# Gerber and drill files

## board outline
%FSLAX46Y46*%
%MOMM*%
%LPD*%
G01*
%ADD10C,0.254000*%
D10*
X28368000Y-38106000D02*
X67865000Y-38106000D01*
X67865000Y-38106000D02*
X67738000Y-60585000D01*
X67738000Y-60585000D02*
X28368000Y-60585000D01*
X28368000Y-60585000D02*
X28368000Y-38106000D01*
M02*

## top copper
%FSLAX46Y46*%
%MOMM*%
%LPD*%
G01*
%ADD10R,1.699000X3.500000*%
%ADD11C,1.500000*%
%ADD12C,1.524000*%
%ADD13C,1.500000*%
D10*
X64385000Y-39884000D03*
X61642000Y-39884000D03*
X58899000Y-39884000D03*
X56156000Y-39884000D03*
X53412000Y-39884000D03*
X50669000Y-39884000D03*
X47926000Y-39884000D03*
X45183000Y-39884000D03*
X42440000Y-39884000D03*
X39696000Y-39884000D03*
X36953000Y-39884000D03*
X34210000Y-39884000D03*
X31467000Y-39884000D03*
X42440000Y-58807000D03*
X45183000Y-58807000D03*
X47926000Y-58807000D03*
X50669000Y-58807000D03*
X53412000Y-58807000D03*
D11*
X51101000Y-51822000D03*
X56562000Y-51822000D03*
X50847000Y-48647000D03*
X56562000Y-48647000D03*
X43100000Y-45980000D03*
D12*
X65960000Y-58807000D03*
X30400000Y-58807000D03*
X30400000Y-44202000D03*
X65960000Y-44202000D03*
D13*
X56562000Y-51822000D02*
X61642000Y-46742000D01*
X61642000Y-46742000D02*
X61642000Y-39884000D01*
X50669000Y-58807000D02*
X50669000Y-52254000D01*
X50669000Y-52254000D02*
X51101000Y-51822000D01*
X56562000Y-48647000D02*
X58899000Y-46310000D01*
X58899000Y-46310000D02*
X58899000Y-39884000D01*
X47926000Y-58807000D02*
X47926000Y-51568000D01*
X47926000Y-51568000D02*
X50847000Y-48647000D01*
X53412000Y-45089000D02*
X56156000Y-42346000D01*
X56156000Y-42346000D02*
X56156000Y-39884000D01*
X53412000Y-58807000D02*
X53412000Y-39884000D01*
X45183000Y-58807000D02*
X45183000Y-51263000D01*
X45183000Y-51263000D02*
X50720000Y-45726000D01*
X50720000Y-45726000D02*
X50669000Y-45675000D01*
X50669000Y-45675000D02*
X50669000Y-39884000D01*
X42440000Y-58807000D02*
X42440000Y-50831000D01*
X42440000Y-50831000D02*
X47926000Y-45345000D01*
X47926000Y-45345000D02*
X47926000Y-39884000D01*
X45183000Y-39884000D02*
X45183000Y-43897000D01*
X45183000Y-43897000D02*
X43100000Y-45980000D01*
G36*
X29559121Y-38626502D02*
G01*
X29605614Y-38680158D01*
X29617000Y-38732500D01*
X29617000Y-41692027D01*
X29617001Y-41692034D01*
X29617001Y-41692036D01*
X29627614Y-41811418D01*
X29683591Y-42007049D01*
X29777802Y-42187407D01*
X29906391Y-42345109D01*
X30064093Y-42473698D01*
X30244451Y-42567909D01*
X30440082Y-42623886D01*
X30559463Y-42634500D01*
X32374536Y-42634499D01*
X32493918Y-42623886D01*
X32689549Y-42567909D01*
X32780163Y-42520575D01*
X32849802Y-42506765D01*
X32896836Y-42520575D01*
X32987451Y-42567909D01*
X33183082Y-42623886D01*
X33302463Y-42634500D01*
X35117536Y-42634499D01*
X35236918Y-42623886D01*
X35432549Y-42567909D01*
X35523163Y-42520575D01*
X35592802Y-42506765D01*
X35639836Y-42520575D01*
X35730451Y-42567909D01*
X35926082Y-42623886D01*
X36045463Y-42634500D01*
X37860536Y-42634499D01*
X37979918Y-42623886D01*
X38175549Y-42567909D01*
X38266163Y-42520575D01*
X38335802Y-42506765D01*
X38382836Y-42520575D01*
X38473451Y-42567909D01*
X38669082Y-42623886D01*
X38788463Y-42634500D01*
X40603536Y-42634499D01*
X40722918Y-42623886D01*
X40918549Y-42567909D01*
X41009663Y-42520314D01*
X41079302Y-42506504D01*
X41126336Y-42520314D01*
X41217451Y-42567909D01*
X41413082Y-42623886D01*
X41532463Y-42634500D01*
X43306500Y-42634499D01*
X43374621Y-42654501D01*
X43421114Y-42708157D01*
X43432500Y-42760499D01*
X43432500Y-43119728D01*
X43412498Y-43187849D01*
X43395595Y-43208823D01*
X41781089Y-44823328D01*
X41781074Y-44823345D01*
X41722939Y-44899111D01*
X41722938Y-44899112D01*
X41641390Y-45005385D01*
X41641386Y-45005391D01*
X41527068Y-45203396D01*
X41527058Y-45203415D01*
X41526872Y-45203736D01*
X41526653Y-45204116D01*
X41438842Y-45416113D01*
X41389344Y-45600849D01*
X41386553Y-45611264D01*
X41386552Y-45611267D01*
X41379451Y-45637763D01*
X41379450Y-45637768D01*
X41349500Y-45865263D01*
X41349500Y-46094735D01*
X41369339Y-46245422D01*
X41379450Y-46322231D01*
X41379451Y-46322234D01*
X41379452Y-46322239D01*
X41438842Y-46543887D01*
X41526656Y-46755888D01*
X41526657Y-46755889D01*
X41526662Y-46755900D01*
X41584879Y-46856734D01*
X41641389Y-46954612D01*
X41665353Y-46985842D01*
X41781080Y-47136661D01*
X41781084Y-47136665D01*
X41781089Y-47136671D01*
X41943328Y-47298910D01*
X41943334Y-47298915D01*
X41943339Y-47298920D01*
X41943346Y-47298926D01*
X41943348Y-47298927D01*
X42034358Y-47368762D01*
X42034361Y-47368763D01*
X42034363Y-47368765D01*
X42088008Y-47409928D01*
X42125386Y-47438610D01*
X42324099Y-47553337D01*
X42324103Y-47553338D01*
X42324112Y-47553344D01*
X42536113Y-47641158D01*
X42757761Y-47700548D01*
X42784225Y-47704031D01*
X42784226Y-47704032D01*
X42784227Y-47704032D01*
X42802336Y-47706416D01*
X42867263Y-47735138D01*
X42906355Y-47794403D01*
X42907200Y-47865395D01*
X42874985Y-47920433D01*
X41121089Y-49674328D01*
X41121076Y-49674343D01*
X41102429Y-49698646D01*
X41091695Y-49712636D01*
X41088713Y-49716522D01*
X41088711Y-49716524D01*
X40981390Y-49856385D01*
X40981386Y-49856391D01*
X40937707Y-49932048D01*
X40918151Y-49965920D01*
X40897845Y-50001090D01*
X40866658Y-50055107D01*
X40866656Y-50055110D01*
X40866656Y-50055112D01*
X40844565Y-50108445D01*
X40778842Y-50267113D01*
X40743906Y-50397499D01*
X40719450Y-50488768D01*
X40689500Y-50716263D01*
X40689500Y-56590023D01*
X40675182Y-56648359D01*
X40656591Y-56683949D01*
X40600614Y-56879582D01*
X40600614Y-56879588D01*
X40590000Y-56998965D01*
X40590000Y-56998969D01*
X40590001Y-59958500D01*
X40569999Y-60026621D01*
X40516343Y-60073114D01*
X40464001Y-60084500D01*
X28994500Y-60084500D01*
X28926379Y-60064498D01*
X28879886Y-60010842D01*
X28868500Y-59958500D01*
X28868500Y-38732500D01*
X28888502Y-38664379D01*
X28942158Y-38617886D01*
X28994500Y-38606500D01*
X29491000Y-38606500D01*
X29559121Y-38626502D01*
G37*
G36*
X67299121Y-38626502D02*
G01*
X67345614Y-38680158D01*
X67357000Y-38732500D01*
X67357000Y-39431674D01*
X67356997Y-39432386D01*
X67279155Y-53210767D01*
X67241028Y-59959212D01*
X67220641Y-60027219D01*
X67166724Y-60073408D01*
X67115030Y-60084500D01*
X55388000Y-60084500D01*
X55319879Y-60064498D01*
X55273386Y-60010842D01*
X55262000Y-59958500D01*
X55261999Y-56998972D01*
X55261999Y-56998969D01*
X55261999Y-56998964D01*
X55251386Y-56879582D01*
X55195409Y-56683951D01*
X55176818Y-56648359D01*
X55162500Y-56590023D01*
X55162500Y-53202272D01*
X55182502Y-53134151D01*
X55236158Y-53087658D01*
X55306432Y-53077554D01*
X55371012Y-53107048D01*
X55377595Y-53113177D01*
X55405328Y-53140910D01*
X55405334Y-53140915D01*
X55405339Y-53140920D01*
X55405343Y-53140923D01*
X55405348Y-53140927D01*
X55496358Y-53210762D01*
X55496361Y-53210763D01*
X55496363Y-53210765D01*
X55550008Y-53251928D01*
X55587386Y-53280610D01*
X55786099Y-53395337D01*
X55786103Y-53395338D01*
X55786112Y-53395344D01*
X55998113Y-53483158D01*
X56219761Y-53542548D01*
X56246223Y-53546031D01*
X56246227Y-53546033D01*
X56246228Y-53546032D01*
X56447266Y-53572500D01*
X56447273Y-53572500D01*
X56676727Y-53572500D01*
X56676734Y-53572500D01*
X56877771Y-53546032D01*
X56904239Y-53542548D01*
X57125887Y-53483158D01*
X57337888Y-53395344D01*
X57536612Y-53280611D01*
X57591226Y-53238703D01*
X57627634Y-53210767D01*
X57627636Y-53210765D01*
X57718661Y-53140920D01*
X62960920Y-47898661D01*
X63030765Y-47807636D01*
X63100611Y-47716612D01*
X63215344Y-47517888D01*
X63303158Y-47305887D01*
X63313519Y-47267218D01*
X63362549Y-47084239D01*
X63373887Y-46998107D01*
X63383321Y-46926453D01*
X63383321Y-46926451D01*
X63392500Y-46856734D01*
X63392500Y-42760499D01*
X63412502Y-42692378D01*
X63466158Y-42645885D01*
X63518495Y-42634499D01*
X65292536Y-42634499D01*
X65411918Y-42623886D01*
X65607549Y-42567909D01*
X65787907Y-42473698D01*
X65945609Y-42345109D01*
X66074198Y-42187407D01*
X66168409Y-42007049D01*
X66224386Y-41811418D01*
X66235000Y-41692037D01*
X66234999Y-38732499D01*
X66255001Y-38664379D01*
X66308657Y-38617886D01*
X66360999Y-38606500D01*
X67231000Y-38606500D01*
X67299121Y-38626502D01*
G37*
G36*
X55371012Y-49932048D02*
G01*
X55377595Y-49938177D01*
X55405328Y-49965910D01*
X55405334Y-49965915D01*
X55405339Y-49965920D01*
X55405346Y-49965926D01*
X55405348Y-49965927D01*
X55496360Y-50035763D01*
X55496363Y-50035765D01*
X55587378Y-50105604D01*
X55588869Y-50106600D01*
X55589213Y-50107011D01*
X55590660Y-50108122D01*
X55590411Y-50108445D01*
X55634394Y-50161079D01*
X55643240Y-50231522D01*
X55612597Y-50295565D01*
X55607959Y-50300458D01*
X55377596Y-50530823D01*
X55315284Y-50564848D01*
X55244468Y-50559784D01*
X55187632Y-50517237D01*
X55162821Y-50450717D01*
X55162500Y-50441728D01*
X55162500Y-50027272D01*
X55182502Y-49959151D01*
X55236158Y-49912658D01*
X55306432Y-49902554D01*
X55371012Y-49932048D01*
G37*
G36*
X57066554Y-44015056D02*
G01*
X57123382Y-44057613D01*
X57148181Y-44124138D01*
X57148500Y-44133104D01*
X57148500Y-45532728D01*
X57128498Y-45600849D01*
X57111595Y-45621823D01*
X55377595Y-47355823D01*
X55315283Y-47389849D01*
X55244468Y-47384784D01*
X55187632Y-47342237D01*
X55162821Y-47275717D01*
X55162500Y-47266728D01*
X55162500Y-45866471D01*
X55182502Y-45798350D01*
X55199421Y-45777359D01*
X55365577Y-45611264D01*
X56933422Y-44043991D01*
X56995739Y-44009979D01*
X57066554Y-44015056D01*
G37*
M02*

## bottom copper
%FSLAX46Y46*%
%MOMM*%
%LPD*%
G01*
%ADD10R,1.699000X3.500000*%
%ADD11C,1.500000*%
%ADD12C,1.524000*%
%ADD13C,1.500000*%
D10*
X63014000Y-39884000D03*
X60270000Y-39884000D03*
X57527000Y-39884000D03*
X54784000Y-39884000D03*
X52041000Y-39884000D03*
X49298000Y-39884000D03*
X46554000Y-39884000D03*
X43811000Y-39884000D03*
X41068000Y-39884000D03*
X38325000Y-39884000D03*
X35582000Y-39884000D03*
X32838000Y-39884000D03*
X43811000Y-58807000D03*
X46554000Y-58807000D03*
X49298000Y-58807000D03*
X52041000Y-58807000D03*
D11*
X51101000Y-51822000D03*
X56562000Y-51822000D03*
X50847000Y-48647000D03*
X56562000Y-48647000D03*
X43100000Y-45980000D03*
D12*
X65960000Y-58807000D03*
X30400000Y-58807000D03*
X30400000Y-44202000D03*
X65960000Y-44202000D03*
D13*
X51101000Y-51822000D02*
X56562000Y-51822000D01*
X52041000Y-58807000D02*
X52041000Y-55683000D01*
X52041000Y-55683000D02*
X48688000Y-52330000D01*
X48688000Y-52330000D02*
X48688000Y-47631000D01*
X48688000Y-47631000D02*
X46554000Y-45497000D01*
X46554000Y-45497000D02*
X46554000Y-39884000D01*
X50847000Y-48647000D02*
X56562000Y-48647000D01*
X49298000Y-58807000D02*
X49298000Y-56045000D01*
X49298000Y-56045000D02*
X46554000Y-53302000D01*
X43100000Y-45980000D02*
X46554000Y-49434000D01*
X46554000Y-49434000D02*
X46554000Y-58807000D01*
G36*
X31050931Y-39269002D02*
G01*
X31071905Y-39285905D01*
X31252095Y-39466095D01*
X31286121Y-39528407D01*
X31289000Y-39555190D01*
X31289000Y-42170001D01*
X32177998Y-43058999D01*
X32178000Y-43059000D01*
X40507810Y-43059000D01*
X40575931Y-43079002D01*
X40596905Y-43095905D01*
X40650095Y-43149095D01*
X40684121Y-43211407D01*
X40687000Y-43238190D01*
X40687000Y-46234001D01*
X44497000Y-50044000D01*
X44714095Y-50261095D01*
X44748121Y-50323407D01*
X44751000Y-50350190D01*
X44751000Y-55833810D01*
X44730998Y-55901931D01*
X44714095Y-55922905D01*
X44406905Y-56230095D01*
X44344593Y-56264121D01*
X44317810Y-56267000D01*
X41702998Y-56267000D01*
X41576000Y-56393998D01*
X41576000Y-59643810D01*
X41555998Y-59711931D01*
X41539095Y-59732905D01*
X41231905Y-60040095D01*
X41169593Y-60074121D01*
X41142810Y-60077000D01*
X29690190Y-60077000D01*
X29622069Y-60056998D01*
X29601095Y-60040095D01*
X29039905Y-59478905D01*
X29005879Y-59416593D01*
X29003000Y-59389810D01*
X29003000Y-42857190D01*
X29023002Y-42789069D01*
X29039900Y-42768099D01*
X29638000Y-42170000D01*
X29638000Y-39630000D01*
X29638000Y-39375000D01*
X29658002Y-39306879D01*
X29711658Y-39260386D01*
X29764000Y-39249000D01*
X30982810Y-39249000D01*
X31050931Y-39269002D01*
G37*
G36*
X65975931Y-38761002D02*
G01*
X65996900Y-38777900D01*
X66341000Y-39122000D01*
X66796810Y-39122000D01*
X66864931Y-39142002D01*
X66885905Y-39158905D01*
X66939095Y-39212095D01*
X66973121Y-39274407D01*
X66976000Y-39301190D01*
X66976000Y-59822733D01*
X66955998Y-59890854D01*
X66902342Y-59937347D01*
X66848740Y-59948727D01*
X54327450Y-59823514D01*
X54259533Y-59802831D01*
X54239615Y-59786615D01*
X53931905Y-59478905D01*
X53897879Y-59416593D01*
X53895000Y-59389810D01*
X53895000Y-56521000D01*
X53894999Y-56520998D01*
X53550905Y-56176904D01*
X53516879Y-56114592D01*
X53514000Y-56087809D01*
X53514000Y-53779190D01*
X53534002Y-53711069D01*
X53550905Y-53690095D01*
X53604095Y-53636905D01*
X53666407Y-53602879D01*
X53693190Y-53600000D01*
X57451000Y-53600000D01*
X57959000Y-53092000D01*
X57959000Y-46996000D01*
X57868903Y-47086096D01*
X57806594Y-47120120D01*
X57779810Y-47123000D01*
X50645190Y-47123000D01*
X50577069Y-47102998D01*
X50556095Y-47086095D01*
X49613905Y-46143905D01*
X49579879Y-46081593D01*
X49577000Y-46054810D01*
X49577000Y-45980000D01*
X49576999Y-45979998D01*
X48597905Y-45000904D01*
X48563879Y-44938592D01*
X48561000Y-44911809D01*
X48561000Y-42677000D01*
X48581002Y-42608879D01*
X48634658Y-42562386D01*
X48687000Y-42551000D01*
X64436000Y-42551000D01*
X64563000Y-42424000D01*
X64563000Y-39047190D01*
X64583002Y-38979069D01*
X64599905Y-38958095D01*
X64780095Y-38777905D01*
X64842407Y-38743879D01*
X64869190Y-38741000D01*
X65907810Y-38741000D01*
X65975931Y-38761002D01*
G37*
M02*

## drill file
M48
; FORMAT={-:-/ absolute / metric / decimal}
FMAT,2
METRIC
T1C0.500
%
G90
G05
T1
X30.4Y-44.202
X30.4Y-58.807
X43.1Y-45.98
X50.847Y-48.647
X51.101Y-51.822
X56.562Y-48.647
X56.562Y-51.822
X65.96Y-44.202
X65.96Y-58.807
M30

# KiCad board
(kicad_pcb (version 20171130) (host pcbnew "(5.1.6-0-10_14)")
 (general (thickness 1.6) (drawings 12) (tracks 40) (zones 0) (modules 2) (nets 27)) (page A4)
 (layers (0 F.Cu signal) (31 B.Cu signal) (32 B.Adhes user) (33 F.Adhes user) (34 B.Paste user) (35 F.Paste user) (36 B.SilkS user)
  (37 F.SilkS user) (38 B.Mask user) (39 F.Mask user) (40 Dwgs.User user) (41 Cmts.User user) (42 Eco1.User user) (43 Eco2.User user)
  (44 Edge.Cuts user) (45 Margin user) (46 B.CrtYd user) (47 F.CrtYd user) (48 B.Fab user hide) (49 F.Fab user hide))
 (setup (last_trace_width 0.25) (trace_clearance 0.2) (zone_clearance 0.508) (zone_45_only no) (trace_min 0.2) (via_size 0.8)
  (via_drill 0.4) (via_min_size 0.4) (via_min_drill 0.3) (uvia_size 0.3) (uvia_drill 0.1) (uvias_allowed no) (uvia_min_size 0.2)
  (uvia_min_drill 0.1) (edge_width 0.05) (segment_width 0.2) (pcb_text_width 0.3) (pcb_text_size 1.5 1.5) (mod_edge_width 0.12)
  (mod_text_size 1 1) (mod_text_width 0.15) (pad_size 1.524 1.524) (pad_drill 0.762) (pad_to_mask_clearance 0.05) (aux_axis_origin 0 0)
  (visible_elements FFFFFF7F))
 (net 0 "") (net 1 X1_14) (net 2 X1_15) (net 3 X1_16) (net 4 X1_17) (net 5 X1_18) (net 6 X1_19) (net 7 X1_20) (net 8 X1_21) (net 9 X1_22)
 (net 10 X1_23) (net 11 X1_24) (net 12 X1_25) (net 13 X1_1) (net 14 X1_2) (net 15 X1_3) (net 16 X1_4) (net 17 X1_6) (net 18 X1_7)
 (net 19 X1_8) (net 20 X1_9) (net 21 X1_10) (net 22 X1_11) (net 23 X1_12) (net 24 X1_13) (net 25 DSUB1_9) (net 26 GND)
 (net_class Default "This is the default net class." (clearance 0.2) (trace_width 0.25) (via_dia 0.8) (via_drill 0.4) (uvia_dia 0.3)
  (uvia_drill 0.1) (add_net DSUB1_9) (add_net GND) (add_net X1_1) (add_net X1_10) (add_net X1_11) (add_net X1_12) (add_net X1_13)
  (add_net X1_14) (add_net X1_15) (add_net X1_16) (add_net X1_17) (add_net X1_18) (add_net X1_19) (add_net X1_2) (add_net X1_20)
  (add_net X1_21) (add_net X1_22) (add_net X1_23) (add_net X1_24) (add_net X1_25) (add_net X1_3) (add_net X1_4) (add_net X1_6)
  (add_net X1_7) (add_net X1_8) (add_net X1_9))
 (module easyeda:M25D (layer F.Cu) (at 47.926 39.884)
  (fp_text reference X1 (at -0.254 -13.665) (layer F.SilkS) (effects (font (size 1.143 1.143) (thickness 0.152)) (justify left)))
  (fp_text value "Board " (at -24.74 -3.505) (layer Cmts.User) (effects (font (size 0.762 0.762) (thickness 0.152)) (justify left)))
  (pad 14 smd rect (at 15.088 0) (size 1.699 3.5) (layers B.Cu B.Paste B.Mask) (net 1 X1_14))
  (pad 15 smd rect (at 12.344 0) (size 1.699 3.5) (layers B.Cu B.Paste B.Mask) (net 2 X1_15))
  (pad 16 smd rect (at 9.601 0) (size 1.699 3.5) (layers B.Cu B.Paste B.Mask) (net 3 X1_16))
  (pad 17 smd rect (at 6.858 0) (size 1.699 3.5) (layers B.Cu B.Paste B.Mask) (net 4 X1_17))
  (pad 18 smd rect (at 4.115 0) (size 1.699 3.5) (layers B.Cu B.Paste B.Mask) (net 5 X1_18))
  (pad 19 smd rect (at 1.372 0) (size 1.699 3.5) (layers B.Cu B.Paste B.Mask) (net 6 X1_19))
  (pad 20 smd rect (at -1.372 0) (size 1.699 3.5) (layers B.Cu B.Paste B.Mask) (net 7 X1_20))
  (pad 21 smd rect (at -4.115 0) (size 1.699 3.5) (layers B.Cu B.Paste B.Mask) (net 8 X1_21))
  (pad 22 smd rect (at -6.858 0) (size 1.699 3.5) (layers B.Cu B.Paste B.Mask) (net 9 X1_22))
  (pad 23 smd rect (at -9.601 0) (size 1.699 3.5) (layers B.Cu B.Paste B.Mask) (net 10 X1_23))
  (pad 24 smd rect (at -12.344 0) (size 1.699 3.5) (layers B.Cu B.Paste B.Mask) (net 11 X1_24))
  (pad 25 smd rect (at -15.088 0) (size 1.699 3.5) (layers B.Cu B.Paste B.Mask) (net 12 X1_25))
  (pad 1 smd rect (at 16.459 0) (size 1.699 3.5) (layers F.Cu F.Paste F.Mask) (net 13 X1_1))
  (pad 2 smd rect (at 13.716 0) (size 1.699 3.5) (layers F.Cu F.Paste F.Mask) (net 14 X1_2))
  (pad 3 smd rect (at 10.973 0) (size 1.699 3.5) (layers F.Cu F.Paste F.Mask) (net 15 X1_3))
  (pad 4 smd rect (at 8.23 0) (size 1.699 3.5) (layers F.Cu F.Paste F.Mask) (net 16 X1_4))
  (pad 5 smd rect (at 5.486 0) (size 1.699 3.5) (layers F.Cu F.Paste F.Mask) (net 16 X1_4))
  (pad 6 smd rect (at 2.743 0) (size 1.699 3.5) (layers F.Cu F.Paste F.Mask) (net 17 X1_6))
  (pad 7 smd rect (at 0 0) (size 1.699 3.5) (layers F.Cu F.Paste F.Mask) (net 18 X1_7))
  (pad 8 smd rect (at -2.743 0) (size 1.699 3.5) (layers F.Cu F.Paste F.Mask) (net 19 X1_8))
  (pad 9 smd rect (at -5.486 0) (size 1.699 3.5) (layers F.Cu F.Paste F.Mask) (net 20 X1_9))
  (pad 10 smd rect (at -8.23 0) (size 1.699 3.5) (layers F.Cu F.Paste F.Mask) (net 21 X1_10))
  (pad 11 smd rect (at -10.973 0) (size 1.699 3.5) (layers F.Cu F.Paste F.Mask) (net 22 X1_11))
  (pad 12 smd rect (at -13.716 0) (size 1.699 3.5) (layers F.Cu F.Paste F.Mask) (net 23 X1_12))
  (pad 13 smd rect (at -16.459 0) (size 1.699 3.5) (layers F.Cu F.Paste F.Mask) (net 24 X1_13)))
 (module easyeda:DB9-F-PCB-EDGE (layer F.Cu) (at 47.926 58.807 180)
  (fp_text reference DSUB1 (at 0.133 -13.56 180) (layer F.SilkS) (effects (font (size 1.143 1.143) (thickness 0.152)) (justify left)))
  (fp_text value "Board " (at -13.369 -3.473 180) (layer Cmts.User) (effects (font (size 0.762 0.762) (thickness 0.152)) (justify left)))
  (pad 9 smd rect (at 4.115 0 180) (size 1.699 3.5) (layers B.Cu B.Paste B.Mask) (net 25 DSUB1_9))
  (pad 8 smd rect (at 1.372 0 180) (size 1.699 3.5) (layers B.Cu B.Paste B.Mask) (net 19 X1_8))
  (pad 7 smd rect (at -1.372 0 180) (size 1.699 3.5) (layers B.Cu B.Paste B.Mask) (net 19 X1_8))
  (pad 6 smd rect (at -4.115 0 180) (size 1.699 3.5) (layers B.Cu B.Paste B.Mask) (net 7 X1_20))
  (pad 5 smd rect (at 5.486 0 180) (size 1.699 3.5) (layers F.Cu F.Paste F.Mask) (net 18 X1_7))
  (pad 4 smd rect (at 2.743 0 180) (size 1.699 3.5) (layers F.Cu F.Paste F.Mask) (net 17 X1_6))
  (pad 3 smd rect (at 0 0 180) (size 1.699 3.5) (layers F.Cu F.Paste F.Mask) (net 15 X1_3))
  (pad 2 smd rect (at -2.743 0 180) (size 1.699 3.5) (layers F.Cu F.Paste F.Mask) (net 14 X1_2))
  (pad 1 smd rect (at -5.486 0 180) (size 1.699 3.5) (layers F.Cu F.Paste F.Mask) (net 16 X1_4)))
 (gr_line (start 28.368 38.106) (end 67.865 38.106) (layer Edge.Cuts) (width 0.254))
 (gr_line (start 67.865 38.106) (end 67.738 60.585) (layer Edge.Cuts) (width 0.254))
 (gr_line (start 67.738 60.585) (end 28.368 60.585) (layer Edge.Cuts) (width 0.254))
 (gr_line (start 28.368 60.585) (end 28.368 38.106) (layer Edge.Cuts) (width 0.254))
 (segment (start 56.562 51.822) (end 61.642 46.742) (width 1.5) (layer F.Cu) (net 14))
 (segment (start 61.642 46.742) (end 61.642 39.884) (width 1.5) (layer F.Cu) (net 14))
 (segment (start 50.669 58.807) (end 50.669 52.254) (width 1.5) (layer F.Cu) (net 14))
 (segment (start 50.669 52.254) (end 51.101 51.822) (width 1.5) (layer F.Cu) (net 14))
 (segment (start 51.101 51.822) (end 56.562 51.822) (width 1.5) (layer B.Cu) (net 14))
 (via (at 51.101 51.822) (size 1.5) (drill 0.5) (layers F.Cu B.Cu) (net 14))
 (via (at 56.562 51.822) (size 1.5) (drill 0.5) (layers F.Cu B.Cu) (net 14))
 (segment (start 52.041 58.807) (end 52.041 55.683) (width 1.5) (layer B.Cu) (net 7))
 (segment (start 52.041 55.683) (end 48.688 52.33) (width 1.5) (layer B.Cu) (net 7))
 (segment (start 48.688 52.33) (end 48.688 47.631) (width 1.5) (layer B.Cu) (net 7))
 (segment (start 48.688 47.631) (end 46.554 45.497) (width 1.5) (layer B.Cu) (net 7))
 (segment (start 46.554 45.497) (end 46.554 39.884) (width 1.5) (layer B.Cu) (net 7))
 (segment (start 56.562 48.647) (end 58.899 46.31) (width 1.5) (layer F.Cu) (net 15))
 (segment (start 58.899 46.31) (end 58.899 39.884) (width 1.5) (layer F.Cu) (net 15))
 (segment (start 47.926 58.807) (end 47.926 51.568) (width 1.5) (layer F.Cu) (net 15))
 (segment (start 47.926 51.568) (end 50.847 48.647) (width 1.5) (layer F.Cu) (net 15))
 (segment (start 50.847 48.647) (end 56.562 48.647) (width 1.5) (layer B.Cu) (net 15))
 (via (at 50.847 48.647) (size 1.5) (drill 0.5) (layers F.Cu B.Cu) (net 15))
 (via (at 56.562 48.647) (size 1.5) (drill 0.5) (layers F.Cu B.Cu) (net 15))
 (segment (start 53.412 45.089) (end 56.156 42.346) (width 1.5) (layer F.Cu) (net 16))
 (segment (start 56.156 42.346) (end 56.156 39.884) (width 1.5) (layer F.Cu) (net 16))
 (segment (start 53.412 58.807) (end 53.412 39.884) (width 1.5) (layer F.Cu) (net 16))
 (segment (start 45.183 58.807) (end 45.183 51.263) (width 1.5) (layer F.Cu) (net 17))
 (segment (start 45.183 51.263) (end 50.72 45.726) (width 1.5) (layer F.Cu) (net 17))
 (segment (start 50.72 45.726) (end 50.669 45.675) (width 1.5) (layer F.Cu) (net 17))
 (segment (start 50.669 45.675) (end 50.669 39.884) (width 1.5) (layer F.Cu) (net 17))
 (segment (start 42.44 58.807) (end 42.44 50.831) (width 1.5) (layer F.Cu) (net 18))
 (segment (start 42.44 50.831) (end 47.926 45.345) (width 1.5) (layer F.Cu) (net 18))
 (segment (start 47.926 45.345) (end 47.926 39.884) (width 1.5) (layer F.Cu) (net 18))
 (segment (start 45.183 39.884) (end 45.183 43.897) (width 1.5) (layer F.Cu) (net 19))
 (segment (start 45.183 43.897) (end 43.1 45.98) (width 1.5) (layer F.Cu) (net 19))
 (segment (start 49.298 58.807) (end 49.298 56.045) (width 1.5) (layer B.Cu) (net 19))
 (segment (start 49.298 56.045) (end 46.554 53.302) (width 1.5) (layer B.Cu) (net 19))
 (segment (start 43.1 45.98) (end 46.554 49.434) (width 1.5) (layer B.Cu) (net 19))
 (segment (start 46.554 49.434) (end 46.554 58.807) (width 1.5) (layer B.Cu) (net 19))
 (via (at 43.1 45.98) (size 1.5) (drill 0.5) (layers F.Cu B.Cu) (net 19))
 (via (at 65.96 58.807) (size 1.524) (drill 0.5) (layers F.Cu B.Cu) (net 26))
 (via (at 30.4 58.807) (size 1.524) (drill 0.5) (layers F.Cu B.Cu) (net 26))
 (via (at 30.4 44.202) (size 1.524) (drill 0.5) (layers F.Cu B.Cu) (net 26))
 (via (at 65.96 44.202) (size 1.524) (drill 0.5) (layers F.Cu B.Cu) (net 26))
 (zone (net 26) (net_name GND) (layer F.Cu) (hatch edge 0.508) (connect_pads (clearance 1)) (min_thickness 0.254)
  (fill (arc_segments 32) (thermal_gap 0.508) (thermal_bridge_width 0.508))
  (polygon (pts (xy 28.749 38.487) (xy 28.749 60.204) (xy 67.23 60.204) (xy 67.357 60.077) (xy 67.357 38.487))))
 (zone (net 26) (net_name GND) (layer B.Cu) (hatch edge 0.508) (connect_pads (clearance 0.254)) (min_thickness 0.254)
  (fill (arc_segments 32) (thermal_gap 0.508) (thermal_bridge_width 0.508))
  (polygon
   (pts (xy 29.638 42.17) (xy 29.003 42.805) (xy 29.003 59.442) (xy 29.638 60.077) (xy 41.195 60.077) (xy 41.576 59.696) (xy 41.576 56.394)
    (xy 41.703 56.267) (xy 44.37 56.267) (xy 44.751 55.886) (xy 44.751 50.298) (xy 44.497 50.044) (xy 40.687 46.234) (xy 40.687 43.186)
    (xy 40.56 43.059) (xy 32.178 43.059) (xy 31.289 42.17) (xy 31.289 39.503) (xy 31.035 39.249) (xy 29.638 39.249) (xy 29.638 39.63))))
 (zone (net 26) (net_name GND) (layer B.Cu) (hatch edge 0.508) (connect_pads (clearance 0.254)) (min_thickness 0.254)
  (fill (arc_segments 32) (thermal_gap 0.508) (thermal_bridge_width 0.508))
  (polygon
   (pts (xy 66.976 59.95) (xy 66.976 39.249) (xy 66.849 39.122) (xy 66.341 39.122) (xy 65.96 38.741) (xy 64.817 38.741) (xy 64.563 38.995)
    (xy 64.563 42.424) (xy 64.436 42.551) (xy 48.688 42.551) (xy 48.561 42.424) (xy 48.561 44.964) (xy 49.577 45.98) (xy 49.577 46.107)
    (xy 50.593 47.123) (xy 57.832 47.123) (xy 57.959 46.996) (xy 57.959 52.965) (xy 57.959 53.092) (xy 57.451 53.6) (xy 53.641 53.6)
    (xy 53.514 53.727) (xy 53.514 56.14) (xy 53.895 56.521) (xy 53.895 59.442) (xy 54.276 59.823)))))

